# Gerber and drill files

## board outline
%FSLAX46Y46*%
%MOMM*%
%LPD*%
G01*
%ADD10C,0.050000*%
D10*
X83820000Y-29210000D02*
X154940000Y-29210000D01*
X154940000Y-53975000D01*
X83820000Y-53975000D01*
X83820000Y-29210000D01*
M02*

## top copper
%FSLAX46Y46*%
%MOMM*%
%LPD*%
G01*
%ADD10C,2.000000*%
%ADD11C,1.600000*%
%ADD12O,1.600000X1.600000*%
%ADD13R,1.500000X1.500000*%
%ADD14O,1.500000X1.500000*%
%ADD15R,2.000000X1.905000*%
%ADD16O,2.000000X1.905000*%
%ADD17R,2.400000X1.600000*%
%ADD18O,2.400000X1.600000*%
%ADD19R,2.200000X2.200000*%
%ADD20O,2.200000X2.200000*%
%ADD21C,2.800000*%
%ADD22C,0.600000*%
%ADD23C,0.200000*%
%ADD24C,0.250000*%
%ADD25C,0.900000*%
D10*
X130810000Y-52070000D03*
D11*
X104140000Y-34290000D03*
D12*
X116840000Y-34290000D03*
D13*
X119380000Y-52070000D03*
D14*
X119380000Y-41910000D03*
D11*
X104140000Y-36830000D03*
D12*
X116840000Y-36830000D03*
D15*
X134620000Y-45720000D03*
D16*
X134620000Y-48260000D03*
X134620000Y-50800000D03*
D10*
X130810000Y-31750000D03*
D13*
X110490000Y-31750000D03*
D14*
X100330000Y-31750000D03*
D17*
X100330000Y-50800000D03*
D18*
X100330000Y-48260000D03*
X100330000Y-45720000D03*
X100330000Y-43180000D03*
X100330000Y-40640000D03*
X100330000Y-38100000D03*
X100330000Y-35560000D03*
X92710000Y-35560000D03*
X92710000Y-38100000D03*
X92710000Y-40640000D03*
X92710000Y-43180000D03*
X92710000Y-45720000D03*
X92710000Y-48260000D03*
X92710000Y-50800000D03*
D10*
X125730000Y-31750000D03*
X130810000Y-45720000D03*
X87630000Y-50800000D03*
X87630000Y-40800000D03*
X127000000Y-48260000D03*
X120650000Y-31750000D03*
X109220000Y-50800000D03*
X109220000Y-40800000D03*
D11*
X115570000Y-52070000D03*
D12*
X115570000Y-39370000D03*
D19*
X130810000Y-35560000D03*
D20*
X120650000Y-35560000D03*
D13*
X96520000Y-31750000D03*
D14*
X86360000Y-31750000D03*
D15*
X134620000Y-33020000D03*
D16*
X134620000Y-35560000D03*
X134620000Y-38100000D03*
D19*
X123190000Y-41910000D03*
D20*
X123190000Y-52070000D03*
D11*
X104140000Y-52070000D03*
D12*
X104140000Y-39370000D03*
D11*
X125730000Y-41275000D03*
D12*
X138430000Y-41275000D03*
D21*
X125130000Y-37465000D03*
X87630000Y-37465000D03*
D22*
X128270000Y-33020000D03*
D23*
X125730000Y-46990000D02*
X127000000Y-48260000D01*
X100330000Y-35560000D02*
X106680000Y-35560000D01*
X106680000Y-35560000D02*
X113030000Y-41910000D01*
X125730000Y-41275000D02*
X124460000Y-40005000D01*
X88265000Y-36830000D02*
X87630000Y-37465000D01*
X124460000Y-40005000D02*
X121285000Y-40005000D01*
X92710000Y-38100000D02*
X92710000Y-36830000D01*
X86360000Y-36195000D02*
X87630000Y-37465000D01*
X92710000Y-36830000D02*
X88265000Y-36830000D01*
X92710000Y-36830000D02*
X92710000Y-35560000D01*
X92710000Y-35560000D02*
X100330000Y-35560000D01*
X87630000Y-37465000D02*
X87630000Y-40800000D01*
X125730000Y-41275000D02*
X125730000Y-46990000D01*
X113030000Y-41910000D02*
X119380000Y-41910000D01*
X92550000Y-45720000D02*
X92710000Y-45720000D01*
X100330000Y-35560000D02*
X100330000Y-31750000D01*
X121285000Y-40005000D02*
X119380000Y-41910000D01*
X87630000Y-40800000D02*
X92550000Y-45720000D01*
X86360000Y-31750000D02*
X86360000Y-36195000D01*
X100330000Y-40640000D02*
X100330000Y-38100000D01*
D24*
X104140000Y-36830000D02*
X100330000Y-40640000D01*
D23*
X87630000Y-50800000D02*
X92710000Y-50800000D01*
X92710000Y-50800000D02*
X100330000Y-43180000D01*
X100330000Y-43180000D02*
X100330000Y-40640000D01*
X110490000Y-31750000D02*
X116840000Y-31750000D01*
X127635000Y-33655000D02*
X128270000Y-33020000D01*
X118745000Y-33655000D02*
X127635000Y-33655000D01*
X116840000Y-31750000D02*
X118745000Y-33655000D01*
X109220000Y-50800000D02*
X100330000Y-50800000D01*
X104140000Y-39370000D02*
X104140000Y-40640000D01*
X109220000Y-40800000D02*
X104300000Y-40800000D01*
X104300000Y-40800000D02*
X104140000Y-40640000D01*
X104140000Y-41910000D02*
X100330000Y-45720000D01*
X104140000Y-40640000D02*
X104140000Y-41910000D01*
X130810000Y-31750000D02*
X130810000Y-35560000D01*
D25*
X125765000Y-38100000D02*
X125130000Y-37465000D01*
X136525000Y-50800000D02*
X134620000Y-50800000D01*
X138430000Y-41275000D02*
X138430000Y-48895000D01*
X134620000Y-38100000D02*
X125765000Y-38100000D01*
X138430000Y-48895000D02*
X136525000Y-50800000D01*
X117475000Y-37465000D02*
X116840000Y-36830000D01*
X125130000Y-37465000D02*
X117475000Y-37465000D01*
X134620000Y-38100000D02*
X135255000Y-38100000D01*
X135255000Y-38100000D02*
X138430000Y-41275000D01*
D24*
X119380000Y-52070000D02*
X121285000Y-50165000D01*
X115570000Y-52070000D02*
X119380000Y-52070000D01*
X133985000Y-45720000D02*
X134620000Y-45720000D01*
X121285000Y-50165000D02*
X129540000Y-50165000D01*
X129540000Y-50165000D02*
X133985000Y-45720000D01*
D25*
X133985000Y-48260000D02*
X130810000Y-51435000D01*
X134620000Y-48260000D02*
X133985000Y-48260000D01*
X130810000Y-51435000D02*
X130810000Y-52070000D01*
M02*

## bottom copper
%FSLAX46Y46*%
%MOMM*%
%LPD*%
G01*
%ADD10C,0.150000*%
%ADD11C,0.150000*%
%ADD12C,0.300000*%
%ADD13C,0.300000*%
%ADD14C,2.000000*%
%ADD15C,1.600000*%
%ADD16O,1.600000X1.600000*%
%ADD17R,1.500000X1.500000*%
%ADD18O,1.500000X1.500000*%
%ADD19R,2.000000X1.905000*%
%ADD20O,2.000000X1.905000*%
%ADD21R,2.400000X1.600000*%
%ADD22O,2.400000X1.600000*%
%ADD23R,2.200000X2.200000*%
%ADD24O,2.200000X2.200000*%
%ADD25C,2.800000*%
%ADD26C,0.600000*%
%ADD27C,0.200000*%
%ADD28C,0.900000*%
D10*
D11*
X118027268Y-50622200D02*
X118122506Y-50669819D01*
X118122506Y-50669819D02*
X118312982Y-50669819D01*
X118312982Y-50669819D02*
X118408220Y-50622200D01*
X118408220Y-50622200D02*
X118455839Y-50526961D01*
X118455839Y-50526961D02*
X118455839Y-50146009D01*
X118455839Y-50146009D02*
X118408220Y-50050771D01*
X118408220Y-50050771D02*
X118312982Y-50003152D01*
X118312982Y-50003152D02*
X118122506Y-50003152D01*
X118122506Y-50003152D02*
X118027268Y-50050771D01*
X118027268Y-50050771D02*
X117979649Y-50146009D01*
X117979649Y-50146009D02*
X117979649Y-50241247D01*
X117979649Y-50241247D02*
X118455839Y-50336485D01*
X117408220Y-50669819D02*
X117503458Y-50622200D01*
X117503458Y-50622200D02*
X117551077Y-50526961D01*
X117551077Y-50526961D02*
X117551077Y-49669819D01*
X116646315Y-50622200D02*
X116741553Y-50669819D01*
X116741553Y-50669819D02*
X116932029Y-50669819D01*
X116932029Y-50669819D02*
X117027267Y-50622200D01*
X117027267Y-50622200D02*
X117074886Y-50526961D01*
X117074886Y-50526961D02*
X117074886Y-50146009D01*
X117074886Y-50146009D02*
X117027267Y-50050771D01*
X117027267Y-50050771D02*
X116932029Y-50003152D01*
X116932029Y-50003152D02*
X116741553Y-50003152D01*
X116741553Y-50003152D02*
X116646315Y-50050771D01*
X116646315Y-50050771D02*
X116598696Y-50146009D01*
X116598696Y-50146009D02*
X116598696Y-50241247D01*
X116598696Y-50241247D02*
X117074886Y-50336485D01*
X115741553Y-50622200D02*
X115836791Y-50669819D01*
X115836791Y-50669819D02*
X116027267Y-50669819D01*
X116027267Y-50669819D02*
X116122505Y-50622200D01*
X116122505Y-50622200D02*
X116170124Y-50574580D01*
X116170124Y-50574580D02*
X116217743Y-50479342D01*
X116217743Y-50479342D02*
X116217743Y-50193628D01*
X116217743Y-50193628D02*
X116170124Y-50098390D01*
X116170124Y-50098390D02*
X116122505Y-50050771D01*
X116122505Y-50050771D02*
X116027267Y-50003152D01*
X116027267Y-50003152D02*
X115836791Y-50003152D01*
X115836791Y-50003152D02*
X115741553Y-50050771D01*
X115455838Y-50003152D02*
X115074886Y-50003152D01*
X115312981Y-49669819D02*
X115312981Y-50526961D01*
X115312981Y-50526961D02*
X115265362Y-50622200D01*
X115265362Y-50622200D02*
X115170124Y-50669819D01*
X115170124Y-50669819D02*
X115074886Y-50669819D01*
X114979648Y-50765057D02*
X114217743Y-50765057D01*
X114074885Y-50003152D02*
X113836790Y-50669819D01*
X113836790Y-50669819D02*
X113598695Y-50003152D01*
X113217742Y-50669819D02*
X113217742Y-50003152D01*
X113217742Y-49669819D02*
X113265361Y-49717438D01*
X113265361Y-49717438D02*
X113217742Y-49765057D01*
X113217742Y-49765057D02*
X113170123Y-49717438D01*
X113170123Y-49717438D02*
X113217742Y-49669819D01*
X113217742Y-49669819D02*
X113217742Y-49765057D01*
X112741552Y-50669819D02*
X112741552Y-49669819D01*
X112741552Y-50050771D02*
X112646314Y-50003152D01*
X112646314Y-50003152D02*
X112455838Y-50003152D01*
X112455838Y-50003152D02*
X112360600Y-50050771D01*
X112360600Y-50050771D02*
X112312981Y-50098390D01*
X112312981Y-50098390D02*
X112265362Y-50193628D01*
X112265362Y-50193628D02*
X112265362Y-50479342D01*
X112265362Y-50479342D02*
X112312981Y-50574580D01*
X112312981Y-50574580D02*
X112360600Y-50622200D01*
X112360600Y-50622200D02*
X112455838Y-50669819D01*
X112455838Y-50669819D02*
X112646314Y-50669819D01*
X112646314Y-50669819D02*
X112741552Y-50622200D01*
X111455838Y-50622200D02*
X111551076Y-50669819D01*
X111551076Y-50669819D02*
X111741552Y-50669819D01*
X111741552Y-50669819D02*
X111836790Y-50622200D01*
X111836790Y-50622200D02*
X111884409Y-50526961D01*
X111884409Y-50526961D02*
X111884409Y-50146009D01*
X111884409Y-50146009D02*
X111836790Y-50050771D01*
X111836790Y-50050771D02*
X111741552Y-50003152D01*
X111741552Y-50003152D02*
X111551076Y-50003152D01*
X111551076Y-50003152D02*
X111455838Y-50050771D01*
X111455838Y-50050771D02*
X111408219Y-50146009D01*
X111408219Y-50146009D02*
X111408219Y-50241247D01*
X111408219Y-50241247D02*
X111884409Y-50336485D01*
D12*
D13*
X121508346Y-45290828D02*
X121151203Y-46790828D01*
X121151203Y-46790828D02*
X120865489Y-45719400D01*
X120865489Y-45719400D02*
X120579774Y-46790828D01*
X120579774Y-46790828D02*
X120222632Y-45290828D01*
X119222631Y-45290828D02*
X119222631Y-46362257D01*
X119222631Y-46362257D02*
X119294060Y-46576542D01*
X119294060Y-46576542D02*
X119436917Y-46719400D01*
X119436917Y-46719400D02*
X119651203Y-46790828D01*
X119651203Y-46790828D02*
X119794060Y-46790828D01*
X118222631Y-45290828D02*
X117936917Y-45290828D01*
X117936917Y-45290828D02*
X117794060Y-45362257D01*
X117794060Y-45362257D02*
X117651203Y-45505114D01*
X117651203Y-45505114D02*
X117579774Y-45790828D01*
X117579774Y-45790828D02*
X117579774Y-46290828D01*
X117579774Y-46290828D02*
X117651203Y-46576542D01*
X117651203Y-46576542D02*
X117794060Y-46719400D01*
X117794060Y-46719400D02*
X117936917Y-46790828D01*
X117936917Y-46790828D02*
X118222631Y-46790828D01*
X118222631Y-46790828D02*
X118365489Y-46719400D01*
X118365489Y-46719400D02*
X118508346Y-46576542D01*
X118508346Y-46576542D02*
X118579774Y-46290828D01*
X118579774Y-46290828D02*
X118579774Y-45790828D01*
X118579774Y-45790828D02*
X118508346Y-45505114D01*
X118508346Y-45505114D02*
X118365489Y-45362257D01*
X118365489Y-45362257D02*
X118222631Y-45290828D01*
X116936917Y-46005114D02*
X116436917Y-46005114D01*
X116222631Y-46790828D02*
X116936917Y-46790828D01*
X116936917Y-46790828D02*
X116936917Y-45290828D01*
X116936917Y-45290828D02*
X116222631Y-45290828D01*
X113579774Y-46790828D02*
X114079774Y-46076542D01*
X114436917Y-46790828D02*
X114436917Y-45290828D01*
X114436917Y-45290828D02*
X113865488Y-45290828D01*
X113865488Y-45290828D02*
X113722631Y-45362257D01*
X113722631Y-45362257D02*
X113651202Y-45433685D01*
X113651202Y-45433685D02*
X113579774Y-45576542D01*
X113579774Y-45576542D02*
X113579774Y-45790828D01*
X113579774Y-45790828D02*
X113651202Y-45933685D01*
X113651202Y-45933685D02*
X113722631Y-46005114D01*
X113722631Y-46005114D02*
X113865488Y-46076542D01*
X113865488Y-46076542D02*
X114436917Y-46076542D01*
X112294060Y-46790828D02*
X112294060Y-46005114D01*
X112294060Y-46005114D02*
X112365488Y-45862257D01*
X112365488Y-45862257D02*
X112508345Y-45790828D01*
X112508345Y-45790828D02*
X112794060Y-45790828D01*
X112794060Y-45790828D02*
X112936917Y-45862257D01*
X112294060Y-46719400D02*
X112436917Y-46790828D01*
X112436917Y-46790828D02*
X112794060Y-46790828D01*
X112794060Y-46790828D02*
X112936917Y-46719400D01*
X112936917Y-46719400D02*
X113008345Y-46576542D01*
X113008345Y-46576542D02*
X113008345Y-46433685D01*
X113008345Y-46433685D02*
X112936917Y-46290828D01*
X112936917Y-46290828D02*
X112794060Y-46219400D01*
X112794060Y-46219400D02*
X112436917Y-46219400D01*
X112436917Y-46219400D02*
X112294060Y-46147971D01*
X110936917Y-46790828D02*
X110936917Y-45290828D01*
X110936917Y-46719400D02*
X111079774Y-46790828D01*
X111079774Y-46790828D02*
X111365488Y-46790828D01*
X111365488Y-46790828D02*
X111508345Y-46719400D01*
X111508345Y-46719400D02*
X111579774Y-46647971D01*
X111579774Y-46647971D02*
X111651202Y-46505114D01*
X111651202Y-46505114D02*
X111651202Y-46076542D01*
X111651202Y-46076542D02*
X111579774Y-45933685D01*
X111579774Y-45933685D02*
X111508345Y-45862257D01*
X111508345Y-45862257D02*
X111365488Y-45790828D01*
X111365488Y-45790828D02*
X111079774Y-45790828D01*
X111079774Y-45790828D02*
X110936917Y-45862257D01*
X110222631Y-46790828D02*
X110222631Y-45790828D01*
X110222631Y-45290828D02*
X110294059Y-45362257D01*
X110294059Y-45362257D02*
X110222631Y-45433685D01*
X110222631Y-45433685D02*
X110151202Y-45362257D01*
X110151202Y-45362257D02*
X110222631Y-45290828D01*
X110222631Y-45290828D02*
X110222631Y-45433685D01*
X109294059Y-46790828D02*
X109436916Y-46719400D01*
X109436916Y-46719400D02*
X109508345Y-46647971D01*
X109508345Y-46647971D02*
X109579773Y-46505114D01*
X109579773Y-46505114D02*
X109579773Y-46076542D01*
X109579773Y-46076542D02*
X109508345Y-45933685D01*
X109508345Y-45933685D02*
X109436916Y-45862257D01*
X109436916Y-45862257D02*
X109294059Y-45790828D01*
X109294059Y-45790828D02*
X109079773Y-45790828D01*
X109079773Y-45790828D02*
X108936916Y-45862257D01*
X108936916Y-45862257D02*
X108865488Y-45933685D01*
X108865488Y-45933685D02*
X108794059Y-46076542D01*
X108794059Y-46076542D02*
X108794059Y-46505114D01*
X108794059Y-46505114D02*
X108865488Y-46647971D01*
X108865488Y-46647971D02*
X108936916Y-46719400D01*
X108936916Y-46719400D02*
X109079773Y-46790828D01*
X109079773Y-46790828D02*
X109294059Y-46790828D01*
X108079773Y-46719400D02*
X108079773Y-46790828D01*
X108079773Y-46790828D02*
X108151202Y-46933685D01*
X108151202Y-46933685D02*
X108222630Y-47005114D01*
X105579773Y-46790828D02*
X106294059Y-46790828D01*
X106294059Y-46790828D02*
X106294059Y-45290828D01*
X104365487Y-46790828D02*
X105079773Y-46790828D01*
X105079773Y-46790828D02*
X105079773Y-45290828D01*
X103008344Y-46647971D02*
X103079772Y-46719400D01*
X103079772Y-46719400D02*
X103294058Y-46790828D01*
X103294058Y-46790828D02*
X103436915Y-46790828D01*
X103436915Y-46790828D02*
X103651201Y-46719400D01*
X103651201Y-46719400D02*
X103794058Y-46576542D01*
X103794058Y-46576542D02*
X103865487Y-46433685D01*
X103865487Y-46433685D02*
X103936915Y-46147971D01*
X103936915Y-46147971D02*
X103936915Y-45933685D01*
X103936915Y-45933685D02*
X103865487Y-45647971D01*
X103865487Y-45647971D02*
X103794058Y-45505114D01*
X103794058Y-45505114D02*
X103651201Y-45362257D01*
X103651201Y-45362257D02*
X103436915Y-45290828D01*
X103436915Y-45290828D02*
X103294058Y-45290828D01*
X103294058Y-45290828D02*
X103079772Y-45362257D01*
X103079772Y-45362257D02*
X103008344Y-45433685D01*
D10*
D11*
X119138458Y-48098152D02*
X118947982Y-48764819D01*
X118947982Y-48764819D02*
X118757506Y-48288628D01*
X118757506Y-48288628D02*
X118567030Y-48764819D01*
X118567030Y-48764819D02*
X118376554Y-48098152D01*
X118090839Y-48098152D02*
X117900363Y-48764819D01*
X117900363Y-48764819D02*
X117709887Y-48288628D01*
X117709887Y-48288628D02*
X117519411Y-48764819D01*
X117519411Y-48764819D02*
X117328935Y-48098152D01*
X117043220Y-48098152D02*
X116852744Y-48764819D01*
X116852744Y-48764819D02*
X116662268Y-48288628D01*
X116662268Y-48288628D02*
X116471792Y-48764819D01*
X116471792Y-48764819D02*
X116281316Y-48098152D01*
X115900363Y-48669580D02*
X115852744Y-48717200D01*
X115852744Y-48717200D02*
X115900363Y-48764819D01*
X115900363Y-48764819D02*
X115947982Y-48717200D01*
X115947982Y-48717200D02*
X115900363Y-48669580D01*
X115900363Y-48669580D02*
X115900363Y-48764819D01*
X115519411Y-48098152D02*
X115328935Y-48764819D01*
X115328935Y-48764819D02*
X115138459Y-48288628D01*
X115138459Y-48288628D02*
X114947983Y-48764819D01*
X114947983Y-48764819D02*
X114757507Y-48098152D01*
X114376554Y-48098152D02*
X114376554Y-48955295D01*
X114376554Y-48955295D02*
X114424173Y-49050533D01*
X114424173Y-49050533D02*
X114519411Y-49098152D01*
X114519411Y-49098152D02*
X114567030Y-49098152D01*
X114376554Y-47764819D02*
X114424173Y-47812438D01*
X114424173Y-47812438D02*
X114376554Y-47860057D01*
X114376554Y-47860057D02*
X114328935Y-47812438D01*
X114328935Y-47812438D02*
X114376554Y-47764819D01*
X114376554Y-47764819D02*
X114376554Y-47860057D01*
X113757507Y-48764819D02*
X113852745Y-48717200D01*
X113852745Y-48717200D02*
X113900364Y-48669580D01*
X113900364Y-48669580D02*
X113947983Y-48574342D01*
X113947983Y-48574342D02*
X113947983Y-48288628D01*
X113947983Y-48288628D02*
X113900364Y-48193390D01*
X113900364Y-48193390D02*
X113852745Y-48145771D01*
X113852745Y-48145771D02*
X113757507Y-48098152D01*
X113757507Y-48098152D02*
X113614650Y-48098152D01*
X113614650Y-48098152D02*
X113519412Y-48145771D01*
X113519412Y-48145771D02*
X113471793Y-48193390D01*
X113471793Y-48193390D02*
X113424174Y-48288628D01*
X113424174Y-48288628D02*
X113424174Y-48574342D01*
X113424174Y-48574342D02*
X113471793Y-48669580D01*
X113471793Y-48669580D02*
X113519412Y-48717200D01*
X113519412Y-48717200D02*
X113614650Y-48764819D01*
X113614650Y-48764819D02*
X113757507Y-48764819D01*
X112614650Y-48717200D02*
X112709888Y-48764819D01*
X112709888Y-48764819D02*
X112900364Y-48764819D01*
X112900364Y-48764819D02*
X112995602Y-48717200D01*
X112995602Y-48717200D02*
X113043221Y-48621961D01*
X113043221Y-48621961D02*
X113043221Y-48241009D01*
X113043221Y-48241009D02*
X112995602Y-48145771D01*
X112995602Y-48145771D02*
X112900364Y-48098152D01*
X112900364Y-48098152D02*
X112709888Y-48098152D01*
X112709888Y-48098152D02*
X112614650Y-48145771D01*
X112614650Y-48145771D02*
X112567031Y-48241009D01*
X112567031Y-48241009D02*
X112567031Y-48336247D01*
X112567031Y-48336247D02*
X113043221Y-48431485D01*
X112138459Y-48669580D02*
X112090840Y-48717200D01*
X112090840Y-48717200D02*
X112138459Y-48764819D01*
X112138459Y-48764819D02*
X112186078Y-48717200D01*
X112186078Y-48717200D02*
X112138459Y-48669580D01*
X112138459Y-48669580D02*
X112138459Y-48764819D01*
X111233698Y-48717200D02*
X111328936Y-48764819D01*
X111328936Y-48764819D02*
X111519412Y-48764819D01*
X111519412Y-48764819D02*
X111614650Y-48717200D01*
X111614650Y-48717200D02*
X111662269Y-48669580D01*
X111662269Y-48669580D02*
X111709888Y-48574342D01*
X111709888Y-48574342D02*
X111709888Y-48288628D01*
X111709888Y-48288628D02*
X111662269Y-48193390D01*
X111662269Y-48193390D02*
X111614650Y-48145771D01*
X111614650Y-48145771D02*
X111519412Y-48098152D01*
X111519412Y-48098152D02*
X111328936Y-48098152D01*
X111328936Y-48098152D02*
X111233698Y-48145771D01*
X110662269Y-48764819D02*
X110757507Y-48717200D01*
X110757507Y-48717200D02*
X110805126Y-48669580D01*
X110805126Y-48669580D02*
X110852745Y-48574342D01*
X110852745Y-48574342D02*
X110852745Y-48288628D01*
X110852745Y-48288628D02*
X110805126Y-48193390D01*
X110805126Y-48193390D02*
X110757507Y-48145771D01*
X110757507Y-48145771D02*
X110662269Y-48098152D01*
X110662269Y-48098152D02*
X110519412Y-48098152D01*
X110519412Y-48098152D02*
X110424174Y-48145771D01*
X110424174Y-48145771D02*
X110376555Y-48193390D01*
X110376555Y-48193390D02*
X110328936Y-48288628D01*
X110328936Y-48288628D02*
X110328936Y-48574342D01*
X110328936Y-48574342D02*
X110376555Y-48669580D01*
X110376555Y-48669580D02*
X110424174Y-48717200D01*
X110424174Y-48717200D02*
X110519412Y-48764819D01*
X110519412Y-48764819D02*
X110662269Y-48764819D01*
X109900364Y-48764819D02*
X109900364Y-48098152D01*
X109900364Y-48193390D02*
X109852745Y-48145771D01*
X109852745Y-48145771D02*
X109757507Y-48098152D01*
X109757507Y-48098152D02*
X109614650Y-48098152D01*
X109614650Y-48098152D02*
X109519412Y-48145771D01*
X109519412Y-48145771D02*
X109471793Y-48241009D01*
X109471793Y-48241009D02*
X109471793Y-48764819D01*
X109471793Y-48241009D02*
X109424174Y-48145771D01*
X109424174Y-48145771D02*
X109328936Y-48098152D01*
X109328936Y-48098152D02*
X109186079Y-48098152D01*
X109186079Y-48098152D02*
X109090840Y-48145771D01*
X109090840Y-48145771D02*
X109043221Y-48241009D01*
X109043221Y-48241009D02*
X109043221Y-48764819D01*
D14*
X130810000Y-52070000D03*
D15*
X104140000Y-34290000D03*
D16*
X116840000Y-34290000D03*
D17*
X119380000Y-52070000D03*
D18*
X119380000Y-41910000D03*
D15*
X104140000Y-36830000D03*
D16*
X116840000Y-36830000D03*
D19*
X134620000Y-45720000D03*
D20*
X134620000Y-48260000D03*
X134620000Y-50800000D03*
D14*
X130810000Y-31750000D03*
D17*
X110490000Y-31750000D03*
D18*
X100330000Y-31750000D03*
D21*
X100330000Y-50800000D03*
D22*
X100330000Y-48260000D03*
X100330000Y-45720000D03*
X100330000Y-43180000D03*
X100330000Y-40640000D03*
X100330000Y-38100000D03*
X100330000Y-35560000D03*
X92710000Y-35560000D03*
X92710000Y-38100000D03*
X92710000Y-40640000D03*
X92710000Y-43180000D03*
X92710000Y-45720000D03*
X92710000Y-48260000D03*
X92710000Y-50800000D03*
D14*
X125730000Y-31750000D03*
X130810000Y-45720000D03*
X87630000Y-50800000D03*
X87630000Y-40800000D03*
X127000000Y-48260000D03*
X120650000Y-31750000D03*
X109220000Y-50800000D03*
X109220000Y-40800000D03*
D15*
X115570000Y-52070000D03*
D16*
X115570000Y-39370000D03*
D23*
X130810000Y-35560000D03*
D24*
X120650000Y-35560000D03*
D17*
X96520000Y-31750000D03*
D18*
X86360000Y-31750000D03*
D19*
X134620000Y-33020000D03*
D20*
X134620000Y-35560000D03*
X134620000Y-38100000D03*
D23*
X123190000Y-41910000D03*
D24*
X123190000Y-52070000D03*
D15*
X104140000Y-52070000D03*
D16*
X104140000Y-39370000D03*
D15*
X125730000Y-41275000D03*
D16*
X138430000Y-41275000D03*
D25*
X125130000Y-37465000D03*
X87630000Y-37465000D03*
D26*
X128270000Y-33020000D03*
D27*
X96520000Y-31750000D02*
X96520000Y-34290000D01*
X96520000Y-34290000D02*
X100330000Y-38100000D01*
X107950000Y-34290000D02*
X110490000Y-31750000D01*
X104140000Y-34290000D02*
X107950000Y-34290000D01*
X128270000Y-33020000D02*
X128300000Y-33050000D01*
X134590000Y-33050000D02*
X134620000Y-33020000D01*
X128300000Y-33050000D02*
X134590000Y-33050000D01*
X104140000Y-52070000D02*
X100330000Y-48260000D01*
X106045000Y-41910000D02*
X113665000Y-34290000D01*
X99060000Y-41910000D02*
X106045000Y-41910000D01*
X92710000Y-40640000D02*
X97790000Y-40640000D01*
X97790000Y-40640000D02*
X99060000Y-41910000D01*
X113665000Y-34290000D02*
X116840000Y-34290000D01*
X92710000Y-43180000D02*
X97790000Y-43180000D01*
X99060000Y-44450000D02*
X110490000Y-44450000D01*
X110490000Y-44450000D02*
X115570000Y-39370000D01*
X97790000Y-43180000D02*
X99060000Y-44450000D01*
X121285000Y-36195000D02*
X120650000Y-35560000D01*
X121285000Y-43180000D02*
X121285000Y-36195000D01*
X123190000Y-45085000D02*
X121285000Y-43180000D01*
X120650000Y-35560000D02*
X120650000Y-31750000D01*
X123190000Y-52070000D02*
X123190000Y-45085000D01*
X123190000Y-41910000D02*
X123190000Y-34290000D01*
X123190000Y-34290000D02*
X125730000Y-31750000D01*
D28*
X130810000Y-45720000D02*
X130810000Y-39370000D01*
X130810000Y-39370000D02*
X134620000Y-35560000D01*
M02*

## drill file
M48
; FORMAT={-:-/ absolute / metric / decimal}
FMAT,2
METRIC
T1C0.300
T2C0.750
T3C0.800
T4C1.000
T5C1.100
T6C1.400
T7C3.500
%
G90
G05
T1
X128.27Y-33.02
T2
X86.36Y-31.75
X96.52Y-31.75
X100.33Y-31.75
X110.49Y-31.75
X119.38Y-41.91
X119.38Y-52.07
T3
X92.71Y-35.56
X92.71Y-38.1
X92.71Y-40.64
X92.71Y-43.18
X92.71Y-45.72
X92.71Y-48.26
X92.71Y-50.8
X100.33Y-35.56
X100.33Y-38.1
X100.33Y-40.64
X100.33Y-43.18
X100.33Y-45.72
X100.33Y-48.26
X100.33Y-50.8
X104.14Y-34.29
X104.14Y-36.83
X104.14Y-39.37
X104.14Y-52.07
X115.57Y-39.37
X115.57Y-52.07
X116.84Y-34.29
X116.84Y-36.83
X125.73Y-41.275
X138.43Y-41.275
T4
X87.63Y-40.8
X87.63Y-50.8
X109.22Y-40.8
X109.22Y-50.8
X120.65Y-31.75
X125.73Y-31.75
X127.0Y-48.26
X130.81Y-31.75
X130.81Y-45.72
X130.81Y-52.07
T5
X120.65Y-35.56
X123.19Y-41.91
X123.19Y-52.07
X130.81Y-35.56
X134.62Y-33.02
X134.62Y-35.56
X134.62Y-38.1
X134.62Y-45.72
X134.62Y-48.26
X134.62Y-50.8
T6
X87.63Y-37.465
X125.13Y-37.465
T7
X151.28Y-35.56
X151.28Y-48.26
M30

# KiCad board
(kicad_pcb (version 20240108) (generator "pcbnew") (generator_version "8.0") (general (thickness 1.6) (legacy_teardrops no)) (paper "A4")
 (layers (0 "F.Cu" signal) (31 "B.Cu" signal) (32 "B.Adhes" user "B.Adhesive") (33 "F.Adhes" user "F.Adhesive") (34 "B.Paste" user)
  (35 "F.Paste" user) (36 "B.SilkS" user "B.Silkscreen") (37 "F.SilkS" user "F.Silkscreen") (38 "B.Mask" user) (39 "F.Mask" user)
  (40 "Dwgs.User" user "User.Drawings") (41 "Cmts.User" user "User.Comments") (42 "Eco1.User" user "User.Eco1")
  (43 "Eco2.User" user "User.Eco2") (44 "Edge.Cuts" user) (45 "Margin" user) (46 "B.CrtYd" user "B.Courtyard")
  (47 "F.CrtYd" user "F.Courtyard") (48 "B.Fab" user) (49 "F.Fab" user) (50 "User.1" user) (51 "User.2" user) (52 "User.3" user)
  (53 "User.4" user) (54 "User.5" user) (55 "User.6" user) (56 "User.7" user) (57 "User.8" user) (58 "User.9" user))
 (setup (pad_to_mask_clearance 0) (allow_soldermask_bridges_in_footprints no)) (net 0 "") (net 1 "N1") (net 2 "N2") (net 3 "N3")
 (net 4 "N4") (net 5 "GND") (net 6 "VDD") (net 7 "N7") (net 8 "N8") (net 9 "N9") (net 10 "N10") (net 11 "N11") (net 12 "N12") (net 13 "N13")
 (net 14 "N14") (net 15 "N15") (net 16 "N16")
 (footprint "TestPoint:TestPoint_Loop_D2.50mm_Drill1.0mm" (layer "F.Cu") (at 130.81 52.07)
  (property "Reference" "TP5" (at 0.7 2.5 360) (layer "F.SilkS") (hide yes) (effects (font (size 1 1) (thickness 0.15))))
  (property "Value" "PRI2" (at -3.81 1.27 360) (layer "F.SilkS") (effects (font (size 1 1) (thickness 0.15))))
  (pad "1" thru_hole circle (at 0 0) (size 2 2) (drill 1) (layers "*.Cu" "*.Mask") (remove_unused_layers no) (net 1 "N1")))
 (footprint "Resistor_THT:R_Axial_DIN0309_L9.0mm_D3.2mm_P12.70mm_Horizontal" (layer "F.Cu") (at 104.14 34.29)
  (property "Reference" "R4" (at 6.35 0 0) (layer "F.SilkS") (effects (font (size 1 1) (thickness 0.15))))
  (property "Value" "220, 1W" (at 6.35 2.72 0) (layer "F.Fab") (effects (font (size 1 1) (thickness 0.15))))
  (pad "1" thru_hole circle (at 0 0) (size 1.6 1.6) (drill 0.8) (layers "*.Cu" "*.Mask") (remove_unused_layers no) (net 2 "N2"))
  (pad "2" thru_hole oval (at 12.7 0) (size 1.6 1.6) (drill 0.8) (layers "*.Cu" "*.Mask") (remove_unused_layers no) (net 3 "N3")))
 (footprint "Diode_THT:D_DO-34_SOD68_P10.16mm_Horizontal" (layer "F.Cu") (at 119.38 52.07 90)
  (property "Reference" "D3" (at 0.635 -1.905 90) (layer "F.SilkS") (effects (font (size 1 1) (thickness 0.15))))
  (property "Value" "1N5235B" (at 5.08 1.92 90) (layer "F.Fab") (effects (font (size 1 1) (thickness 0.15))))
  (pad "1" thru_hole rect (at 0 0 90) (size 1.5 1.5) (drill 0.75) (layers "*.Cu" "*.Mask") (remove_unused_layers no) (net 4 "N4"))
  (pad "2" thru_hole oval (at 10.16 0 90) (size 1.5 1.5) (drill 0.75) (layers "*.Cu" "*.Mask") (remove_unused_layers no) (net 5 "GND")))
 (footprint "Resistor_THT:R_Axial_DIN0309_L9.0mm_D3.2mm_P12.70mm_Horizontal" (layer "F.Cu") (at 104.14 36.83)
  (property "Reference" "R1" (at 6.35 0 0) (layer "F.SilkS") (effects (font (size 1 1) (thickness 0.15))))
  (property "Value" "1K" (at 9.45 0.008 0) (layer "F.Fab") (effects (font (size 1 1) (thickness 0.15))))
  (pad "1" thru_hole circle (at 0 0) (size 1.6 1.6) (drill 0.8) (layers "*.Cu" "*.Mask") (remove_unused_layers no) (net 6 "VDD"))
  (pad "2" thru_hole oval (at 12.7 0) (size 1.6 1.6) (drill 0.8) (layers "*.Cu" "*.Mask") (remove_unused_layers no) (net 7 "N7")))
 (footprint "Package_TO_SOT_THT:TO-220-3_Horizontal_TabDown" (layer "F.Cu") (at 134.62 45.72 -90)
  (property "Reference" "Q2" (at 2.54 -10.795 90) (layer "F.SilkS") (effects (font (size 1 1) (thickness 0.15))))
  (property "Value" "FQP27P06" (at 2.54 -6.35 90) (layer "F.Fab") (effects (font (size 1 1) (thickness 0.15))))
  (pad "" np_thru_hole circle (at 2.54 -16.66 270) (size 3.5 3.5) (drill 3.5) (layers "*.Cu" "*.Mask"))
  (pad "1" thru_hole rect (at 0 0 270) (size 1.905 2) (drill 1.1) (layers "*.Cu" "*.Mask") (remove_unused_layers no) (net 4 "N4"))
  (pad "2" thru_hole oval (at 2.54 0 270) (size 1.905 2) (drill 1.1) (layers "*.Cu" "*.Mask") (remove_unused_layers no) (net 1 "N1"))
  (pad "3" thru_hole oval (at 5.08 0 270) (size 1.905 2) (drill 1.1) (layers "*.Cu" "*.Mask") (remove_unused_layers no) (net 7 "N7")))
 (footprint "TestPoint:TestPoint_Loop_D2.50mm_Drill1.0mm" (layer "F.Cu") (at 130.81 31.75)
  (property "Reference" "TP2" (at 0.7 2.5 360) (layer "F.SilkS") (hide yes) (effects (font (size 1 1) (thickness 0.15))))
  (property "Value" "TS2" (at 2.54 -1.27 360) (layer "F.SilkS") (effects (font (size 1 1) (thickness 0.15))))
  (pad "1" thru_hole circle (at 0 0) (size 2 2) (drill 1) (layers "*.Cu" "*.Mask") (remove_unused_layers no) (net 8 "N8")))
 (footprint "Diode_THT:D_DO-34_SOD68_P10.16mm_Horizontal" (layer "F.Cu") (at 110.49 31.75 180)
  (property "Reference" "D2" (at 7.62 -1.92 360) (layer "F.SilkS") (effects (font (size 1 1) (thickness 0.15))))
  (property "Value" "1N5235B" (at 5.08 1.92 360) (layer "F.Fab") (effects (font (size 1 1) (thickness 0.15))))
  (pad "1" thru_hole rect (at 0 0 180) (size 1.5 1.5) (drill 0.75) (layers "*.Cu" "*.Mask") (remove_unused_layers no) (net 2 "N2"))
  (pad "2" thru_hole oval (at 10.16 0 180) (size 1.5 1.5) (drill 0.75) (layers "*.Cu" "*.Mask") (remove_unused_layers no) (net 5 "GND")))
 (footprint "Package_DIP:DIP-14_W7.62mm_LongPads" (layer "F.Cu") (at 100.33 50.8 180)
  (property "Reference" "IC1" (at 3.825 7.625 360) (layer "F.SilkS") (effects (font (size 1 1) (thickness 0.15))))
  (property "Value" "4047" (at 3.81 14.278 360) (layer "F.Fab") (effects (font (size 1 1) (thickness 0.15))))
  (pad "1" thru_hole rect (at 0 0 180) (size 2.4 1.6) (drill 0.8) (layers "*.Cu" "*.Mask") (remove_unused_layers no) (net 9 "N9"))
  (pad "2" thru_hole oval (at 0 2.54 180) (size 2.4 1.6) (drill 0.8) (layers "*.Cu" "*.Mask") (remove_unused_layers no) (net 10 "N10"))
  (pad "3" thru_hole oval (at 0 5.08 180) (size 2.4 1.6) (drill 0.8) (layers "*.Cu" "*.Mask") (remove_unused_layers no) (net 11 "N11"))
  (pad "4" thru_hole oval (at 0 7.62 180) (size 2.4 1.6) (drill 0.8) (layers "*.Cu" "*.Mask") (remove_unused_layers no) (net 6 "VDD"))
  (pad "5" thru_hole oval (at 0 10.16 180) (size 2.4 1.6) (drill 0.8) (layers "*.Cu" "*.Mask") (remove_unused_layers no) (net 6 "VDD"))
  (pad "6" thru_hole oval (at 0 12.7 180) (size 2.4 1.6) (drill 0.8) (layers "*.Cu" "*.Mask") (remove_unused_layers no) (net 6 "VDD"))
  (pad "7" thru_hole oval (at 0 15.24 180) (size 2.4 1.6) (drill 0.8) (layers "*.Cu" "*.Mask") (remove_unused_layers no) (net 5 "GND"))
  (pad "8" thru_hole oval (at 7.62 15.24 180) (size 2.4 1.6) (drill 0.8) (layers "*.Cu" "*.Mask") (remove_unused_layers no) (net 5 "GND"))
  (pad "9" thru_hole oval (at 7.62 12.7 180) (size 2.4 1.6) (drill 0.8) (layers "*.Cu" "*.Mask") (remove_unused_layers no) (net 5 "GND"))
  (pad "10" thru_hole oval (at 7.62 10.16 180) (size 2.4 1.6) (drill 0.8) (layers "*.Cu" "*.Mask") (remove_unused_layers no) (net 3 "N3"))
  (pad "11" thru_hole oval (at 7.62 7.62 180) (size 2.4 1.6) (drill 0.8) (layers "*.Cu" "*.Mask") (remove_unused_layers no) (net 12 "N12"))
  (pad "12" thru_hole oval (at 7.62 5.08 180) (size 2.4 1.6) (drill 0.8) (layers "*.Cu" "*.Mask") (remove_unused_layers no) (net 5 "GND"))
  (pad "13" thru_hole oval (at 7.62 2.54 180) (size 2.4 1.6) (drill 0.8) (layers "*.Cu" "*.Mask") (remove_unused_layers no) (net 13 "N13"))
  (pad "14" thru_hole oval (at 7.62 0 180) (size 2.4 1.6) (drill 0.8) (layers "*.Cu" "*.Mask") (remove_unused_layers no) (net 6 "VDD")))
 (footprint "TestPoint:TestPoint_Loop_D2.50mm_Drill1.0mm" (layer "F.Cu") (at 125.73 31.75 90)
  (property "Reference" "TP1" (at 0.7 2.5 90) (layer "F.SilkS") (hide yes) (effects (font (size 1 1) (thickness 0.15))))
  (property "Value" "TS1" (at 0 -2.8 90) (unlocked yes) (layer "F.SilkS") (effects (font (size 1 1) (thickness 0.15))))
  (pad "1" thru_hole circle (at 0 0 90) (size 2 2) (drill 1) (layers "*.Cu" "*.Mask") (remove_unused_layers no) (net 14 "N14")))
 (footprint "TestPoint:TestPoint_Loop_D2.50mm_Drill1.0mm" (layer "F.Cu") (at 130.81 45.72)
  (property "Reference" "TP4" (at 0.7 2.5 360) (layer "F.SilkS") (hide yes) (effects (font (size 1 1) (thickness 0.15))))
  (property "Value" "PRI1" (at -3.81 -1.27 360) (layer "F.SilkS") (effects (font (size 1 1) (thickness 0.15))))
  (pad "1" thru_hole circle (at 0 0) (size 2 2) (drill 1) (layers "*.Cu" "*.Mask") (remove_unused_layers no) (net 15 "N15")))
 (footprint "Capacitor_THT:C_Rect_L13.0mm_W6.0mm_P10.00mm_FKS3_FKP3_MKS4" (layer "F.Cu") (at 87.63 50.8 90)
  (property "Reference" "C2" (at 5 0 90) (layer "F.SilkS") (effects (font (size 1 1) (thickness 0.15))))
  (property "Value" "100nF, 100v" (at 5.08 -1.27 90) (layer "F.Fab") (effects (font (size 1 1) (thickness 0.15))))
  (pad "1" thru_hole circle (at 0 0 90) (size 2 2) (drill 1) (layers "*.Cu" "*.Mask") (remove_unused_layers no) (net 6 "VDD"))
  (pad "2" thru_hole circle (at 10 0 90) (size 2 2) (drill 1) (layers "*.Cu" "*.Mask") (remove_unused_layers no) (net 5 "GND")))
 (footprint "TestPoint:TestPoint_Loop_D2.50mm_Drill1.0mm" (layer "F.Cu") (at 127 48.26)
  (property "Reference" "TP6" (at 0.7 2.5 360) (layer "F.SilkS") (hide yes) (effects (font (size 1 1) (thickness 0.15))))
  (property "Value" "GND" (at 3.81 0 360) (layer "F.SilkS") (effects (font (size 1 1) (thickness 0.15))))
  (pad "1" thru_hole circle (at 0 0) (size 2 2) (drill 1) (layers "*.Cu" "*.Mask") (remove_unused_layers no) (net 5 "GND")))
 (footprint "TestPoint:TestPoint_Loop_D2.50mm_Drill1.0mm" (layer "F.Cu") (at 120.65 31.75)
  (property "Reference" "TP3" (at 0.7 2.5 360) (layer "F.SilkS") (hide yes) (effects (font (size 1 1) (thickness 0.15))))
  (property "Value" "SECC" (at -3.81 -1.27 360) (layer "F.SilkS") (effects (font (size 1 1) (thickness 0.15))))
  (pad "1" thru_hole circle (at 0 0) (size 2 2) (drill 1) (layers "*.Cu" "*.Mask") (remove_unused_layers no) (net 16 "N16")))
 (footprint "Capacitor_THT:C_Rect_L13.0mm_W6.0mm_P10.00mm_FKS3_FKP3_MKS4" (layer "F.Cu") (at 109.22 50.8 90)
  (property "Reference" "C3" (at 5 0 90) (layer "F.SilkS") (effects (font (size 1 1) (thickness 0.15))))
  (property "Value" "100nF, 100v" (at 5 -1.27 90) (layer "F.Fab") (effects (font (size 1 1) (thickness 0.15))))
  (pad "1" thru_hole circle (at 0 0 90) (size 2 2) (drill 1) (layers "*.Cu" "*.Mask") (remove_unused_layers no) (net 9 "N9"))
  (pad "2" thru_hole circle (at 10 0 90) (size 2 2) (drill 1) (layers "*.Cu" "*.Mask") (remove_unused_layers no) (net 11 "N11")))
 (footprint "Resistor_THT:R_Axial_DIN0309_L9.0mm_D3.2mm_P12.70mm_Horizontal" (layer "F.Cu") (at 115.57 52.07 90)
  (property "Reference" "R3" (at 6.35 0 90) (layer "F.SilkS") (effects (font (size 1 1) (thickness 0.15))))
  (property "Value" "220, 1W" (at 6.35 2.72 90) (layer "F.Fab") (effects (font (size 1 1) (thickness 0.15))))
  (pad "1" thru_hole circle (at 0 0 90) (size 1.6 1.6) (drill 0.8) (layers "*.Cu" "*.Mask") (remove_unused_layers no) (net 4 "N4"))
  (pad "2" thru_hole oval (at 12.7 0 90) (size 1.6 1.6) (drill 0.8) (layers "*.Cu" "*.Mask") (remove_unused_layers no) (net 12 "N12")))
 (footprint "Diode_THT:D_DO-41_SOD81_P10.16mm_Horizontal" (layer "F.Cu") (at 130.81 35.56 180)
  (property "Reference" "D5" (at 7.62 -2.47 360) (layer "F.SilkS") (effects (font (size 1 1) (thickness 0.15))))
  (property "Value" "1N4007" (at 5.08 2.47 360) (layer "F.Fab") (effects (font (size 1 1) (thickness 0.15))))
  (pad "1" thru_hole rect (at 0 0 180) (size 2.2 2.2) (drill 1.1) (layers "*.Cu" "*.Mask") (remove_unused_layers no) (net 8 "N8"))
  (pad "2" thru_hole oval (at 10.16 0 180) (size 2.2 2.2) (drill 1.1) (layers "*.Cu" "*.Mask") (remove_unused_layers no) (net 16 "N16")))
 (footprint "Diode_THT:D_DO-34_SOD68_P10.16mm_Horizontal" (layer "F.Cu") (at 96.52 31.75 180)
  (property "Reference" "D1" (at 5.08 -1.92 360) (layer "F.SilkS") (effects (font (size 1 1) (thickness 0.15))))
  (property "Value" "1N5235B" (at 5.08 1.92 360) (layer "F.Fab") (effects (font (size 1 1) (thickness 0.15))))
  (pad "1" thru_hole rect (at 0 0 180) (size 1.5 1.5) (drill 0.75) (layers "*.Cu" "*.Mask") (remove_unused_layers no) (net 6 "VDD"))
  (pad "2" thru_hole oval (at 10.16 0 180) (size 1.5 1.5) (drill 0.75) (layers "*.Cu" "*.Mask") (remove_unused_layers no) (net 5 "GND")))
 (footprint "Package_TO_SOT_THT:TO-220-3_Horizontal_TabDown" (layer "F.Cu") (at 134.62 33.02 -90)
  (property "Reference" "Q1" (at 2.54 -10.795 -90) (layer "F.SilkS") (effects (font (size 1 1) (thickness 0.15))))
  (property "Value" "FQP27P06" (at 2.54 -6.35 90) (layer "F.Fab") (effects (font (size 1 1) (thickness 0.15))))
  (pad "" np_thru_hole circle (at 2.54 -16.66 270) (size 3.5 3.5) (drill 3.5) (layers "*.Cu" "*.Mask"))
  (pad "1" thru_hole rect (at 0 0 270) (size 1.905 2) (drill 1.1) (layers "*.Cu" "*.Mask") (remove_unused_layers no) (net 2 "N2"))
  (pad "2" thru_hole oval (at 2.54 0 270) (size 1.905 2) (drill 1.1) (layers "*.Cu" "*.Mask") (remove_unused_layers no) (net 15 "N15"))
  (pad "3" thru_hole oval (at 5.08 0 270) (size 1.905 2) (drill 1.1) (layers "*.Cu" "*.Mask") (remove_unused_layers no) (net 7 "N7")))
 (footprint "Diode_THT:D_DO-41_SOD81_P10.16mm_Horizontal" (layer "F.Cu") (at 123.19 41.91 -90)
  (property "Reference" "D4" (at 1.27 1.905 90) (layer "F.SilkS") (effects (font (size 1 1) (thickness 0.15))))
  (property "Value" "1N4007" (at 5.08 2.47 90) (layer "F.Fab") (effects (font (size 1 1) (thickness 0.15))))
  (pad "1" thru_hole rect (at 0 0 270) (size 2.2 2.2) (drill 1.1) (layers "*.Cu" "*.Mask") (remove_unused_layers no) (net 14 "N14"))
  (pad "2" thru_hole oval (at 10.16 0 270) (size 2.2 2.2) (drill 1.1) (layers "*.Cu" "*.Mask") (remove_unused_layers no) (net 16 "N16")))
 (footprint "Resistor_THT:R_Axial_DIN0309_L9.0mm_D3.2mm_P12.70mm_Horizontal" (layer "F.Cu") (at 104.14 52.07 90)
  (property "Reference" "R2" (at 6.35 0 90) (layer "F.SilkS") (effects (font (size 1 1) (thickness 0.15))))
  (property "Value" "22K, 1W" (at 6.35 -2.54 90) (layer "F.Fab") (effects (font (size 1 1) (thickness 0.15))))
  (pad "1" thru_hole circle (at 0 0 90) (size 1.6 1.6) (drill 0.8) (layers "*.Cu" "*.Mask") (remove_unused_layers no) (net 10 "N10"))
  (pad "2" thru_hole oval (at 12.7 0 90) (size 1.6 1.6) (drill 0.8) (layers "*.Cu" "*.Mask") (remove_unused_layers no) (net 11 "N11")))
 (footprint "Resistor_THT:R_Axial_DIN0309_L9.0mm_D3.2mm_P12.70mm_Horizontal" (layer "F.Cu") (at 125.73 41.275)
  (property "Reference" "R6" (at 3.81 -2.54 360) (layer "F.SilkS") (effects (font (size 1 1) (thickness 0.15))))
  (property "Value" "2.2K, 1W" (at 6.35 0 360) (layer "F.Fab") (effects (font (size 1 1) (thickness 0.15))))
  (pad "1" thru_hole circle (at 0 0) (size 1.6 1.6) (drill 0.8) (layers "*.Cu" "*.Mask") (remove_unused_layers no) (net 5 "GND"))
  (pad "2" thru_hole oval (at 12.7 0) (size 1.6 1.6) (drill 0.8) (layers "*.Cu" "*.Mask") (remove_unused_layers no) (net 7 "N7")))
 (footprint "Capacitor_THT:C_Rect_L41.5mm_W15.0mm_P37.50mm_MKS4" (layer "B.Cu") (at 125.13 37.465 180)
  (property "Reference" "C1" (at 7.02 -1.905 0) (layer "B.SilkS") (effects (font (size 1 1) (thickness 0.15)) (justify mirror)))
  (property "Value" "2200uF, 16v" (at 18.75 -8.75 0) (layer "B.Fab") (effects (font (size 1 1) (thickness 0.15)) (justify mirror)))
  (pad "1" thru_hole circle (at 0 0 180) (size 2.8 2.8) (drill 1.4) (layers "*.Cu" "*.Mask") (remove_unused_layers no) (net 7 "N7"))
  (pad "2" thru_hole circle (at 37.5 0 180) (size 2.8 2.8) (drill 1.4) (layers "*.Cu" "*.Mask") (remove_unused_layers no) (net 5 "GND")))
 (gr_rect (start 83.82 29.21) (end 154.94 53.975) (stroke (width 0.05) (type default)) (fill none) (layer "Edge.Cuts"))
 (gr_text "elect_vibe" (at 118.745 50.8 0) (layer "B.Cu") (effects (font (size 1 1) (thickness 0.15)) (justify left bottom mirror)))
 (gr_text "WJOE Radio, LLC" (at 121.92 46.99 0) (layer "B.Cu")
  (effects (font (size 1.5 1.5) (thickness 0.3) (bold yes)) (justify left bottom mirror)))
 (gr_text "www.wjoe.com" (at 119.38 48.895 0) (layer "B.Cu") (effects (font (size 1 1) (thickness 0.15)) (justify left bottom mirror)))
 (segment (start 125.73 46.99) (end 127 48.26) (width 0.2) (layer "F.Cu") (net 5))
 (segment (start 100.33 35.56) (end 106.68 35.56) (width 0.2) (layer "F.Cu") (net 5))
 (segment (start 106.68 35.56) (end 113.03 41.91) (width 0.2) (layer "F.Cu") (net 5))
 (segment (start 125.73 41.275) (end 124.46 40.005) (width 0.2) (layer "F.Cu") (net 5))
 (segment (start 88.265 36.83) (end 87.63 37.465) (width 0.2) (layer "F.Cu") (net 5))
 (segment (start 124.46 40.005) (end 121.285 40.005) (width 0.2) (layer "F.Cu") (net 5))
 (segment (start 92.71 38.1) (end 92.71 36.83) (width 0.2) (layer "F.Cu") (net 5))
 (segment (start 86.36 36.195) (end 87.63 37.465) (width 0.2) (layer "F.Cu") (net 5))
 (segment (start 92.71 36.83) (end 88.265 36.83) (width 0.2) (layer "F.Cu") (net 5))
 (segment (start 92.71 36.83) (end 92.71 35.56) (width 0.2) (layer "F.Cu") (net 5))
 (segment (start 92.71 35.56) (end 100.33 35.56) (width 0.2) (layer "F.Cu") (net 5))
 (segment (start 87.63 37.465) (end 87.63 40.8) (width 0.2) (layer "F.Cu") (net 5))
 (segment (start 125.73 41.275) (end 125.73 46.99) (width 0.2) (layer "F.Cu") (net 5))
 (segment (start 113.03 41.91) (end 119.38 41.91) (width 0.2) (layer "F.Cu") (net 5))
 (segment (start 92.55 45.72) (end 92.71 45.72) (width 0.2) (layer "F.Cu") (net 5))
 (segment (start 100.33 35.56) (end 100.33 31.75) (width 0.2) (layer "F.Cu") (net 5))
 (segment (start 121.285 40.005) (end 119.38 41.91) (width 0.2) (layer "F.Cu") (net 5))
 (segment (start 87.63 40.8) (end 92.55 45.72) (width 0.2) (layer "F.Cu") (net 5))
 (segment (start 86.36 31.75) (end 86.36 36.195) (width 0.2) (layer "F.Cu") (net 5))
 (segment (start 100.33 40.64) (end 100.33 38.1) (width 0.2) (layer "F.Cu") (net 6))
 (segment (start 104.14 36.83) (end 100.33 40.64) (width 0.25) (layer "F.Cu") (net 6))
 (segment (start 87.63 50.8) (end 92.71 50.8) (width 0.2) (layer "F.Cu") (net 6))
 (segment (start 92.71 50.8) (end 100.33 43.18) (width 0.2) (layer "F.Cu") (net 6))
 (segment (start 100.33 43.18) (end 100.33 40.64) (width 0.2) (layer "F.Cu") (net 6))
 (segment (start 96.52 31.75) (end 96.52 34.29) (width 0.2) (layer "B.Cu") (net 6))
 (segment (start 96.52 34.29) (end 100.33 38.1) (width 0.2) (layer "B.Cu") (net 6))
 (segment (start 110.49 31.75) (end 116.84 31.75) (width 0.2) (layer "F.Cu") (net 2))
 (segment (start 127.635 33.655) (end 128.27 33.02) (width 0.2) (layer "F.Cu") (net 2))
 (segment (start 118.745 33.655) (end 127.635 33.655) (width 0.2) (layer "F.Cu") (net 2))
 (segment (start 116.84 31.75) (end 118.745 33.655) (width 0.2) (layer "F.Cu") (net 2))
 (via (at 128.27 33.02) (size 0.6) (drill 0.3) (layers "F.Cu" "B.Cu") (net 2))
 (segment (start 107.95 34.29) (end 110.49 31.75) (width 0.2) (layer "B.Cu") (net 2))
 (segment (start 104.14 34.29) (end 107.95 34.29) (width 0.2) (layer "B.Cu") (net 2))
 (segment (start 128.27 33.02) (end 128.3 33.05) (width 0.2) (layer "B.Cu") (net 2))
 (segment (start 134.59 33.05) (end 134.62 33.02) (width 0.2) (layer "B.Cu") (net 2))
 (segment (start 128.3 33.05) (end 134.59 33.05) (width 0.2) (layer "B.Cu") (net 2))
 (segment (start 109.22 50.8) (end 100.33 50.8) (width 0.2) (layer "F.Cu") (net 9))
 (segment (start 104.14 39.37) (end 104.14 40.64) (width 0.2) (layer "F.Cu") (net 11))
 (segment (start 109.22 40.8) (end 104.3 40.8) (width 0.2) (layer "F.Cu") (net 11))
 (segment (start 104.3 40.8) (end 104.14 40.64) (width 0.2) (layer "F.Cu") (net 11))
 (segment (start 104.14 41.91) (end 100.33 45.72) (width 0.2) (layer "F.Cu") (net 11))
 (segment (start 104.14 40.64) (end 104.14 41.91) (width 0.2) (layer "F.Cu") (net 11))
 (segment (start 104.14 52.07) (end 100.33 48.26) (width 0.2) (layer "B.Cu") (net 10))
 (segment (start 106.045 41.91) (end 113.665 34.29) (width 0.2) (layer "B.Cu") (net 3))
 (segment (start 99.06 41.91) (end 106.045 41.91) (width 0.2) (layer "B.Cu") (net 3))
 (segment (start 92.71 40.64) (end 97.79 40.64) (width 0.2) (layer "B.Cu") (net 3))
 (segment (start 97.79 40.64) (end 99.06 41.91) (width 0.2) (layer "B.Cu") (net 3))
 (segment (start 113.665 34.29) (end 116.84 34.29) (width 0.2) (layer "B.Cu") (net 3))
 (segment (start 92.71 43.18) (end 97.79 43.18) (width 0.2) (layer "B.Cu") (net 12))
 (segment (start 99.06 44.45) (end 110.49 44.45) (width 0.2) (layer "B.Cu") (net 12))
 (segment (start 110.49 44.45) (end 115.57 39.37) (width 0.2) (layer "B.Cu") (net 12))
 (segment (start 97.79 43.18) (end 99.06 44.45) (width 0.2) (layer "B.Cu") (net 12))
 (segment (start 121.285 36.195) (end 120.65 35.56) (width 0.2) (layer "B.Cu") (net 16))
 (segment (start 121.285 43.18) (end 121.285 36.195) (width 0.2) (layer "B.Cu") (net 16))
 (segment (start 123.19 45.085) (end 121.285 43.18) (width 0.2) (layer "B.Cu") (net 16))
 (segment (start 120.65 35.56) (end 120.65 31.75) (width 0.2) (layer "B.Cu") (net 16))
 (segment (start 123.19 52.07) (end 123.19 45.085) (width 0.2) (layer "B.Cu") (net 16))
 (segment (start 123.19 41.91) (end 123.19 34.29) (width 0.2) (layer "B.Cu") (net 14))
 (segment (start 123.19 34.29) (end 125.73 31.75) (width 0.2) (layer "B.Cu") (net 14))
 (segment (start 130.81 31.75) (end 130.81 35.56) (width 0.2) (layer "F.Cu") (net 8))
 (segment (start 125.765 38.1) (end 125.13 37.465) (width 0.9) (layer "F.Cu") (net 7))
 (segment (start 136.525 50.8) (end 134.62 50.8) (width 0.9) (layer "F.Cu") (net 7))
 (segment (start 138.43 41.275) (end 138.43 48.895) (width 0.9) (layer "F.Cu") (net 7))
 (segment (start 134.62 38.1) (end 125.765 38.1) (width 0.9) (layer "F.Cu") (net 7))
 (segment (start 138.43 48.895) (end 136.525 50.8) (width 0.9) (layer "F.Cu") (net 7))
 (segment (start 117.475 37.465) (end 116.84 36.83) (width 0.9) (layer "F.Cu") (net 7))
 (segment (start 125.13 37.465) (end 117.475 37.465) (width 0.9) (layer "F.Cu") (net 7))
 (segment (start 134.62 38.1) (end 135.255 38.1) (width 0.9) (layer "F.Cu") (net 7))
 (segment (start 135.255 38.1) (end 138.43 41.275) (width 0.9) (layer "F.Cu") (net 7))
 (segment (start 119.38 52.07) (end 121.285 50.165) (width 0.25) (layer "F.Cu") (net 4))
 (segment (start 115.57 52.07) (end 119.38 52.07) (width 0.25) (layer "F.Cu") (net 4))
 (segment (start 133.985 45.72) (end 134.62 45.72) (width 0.25) (layer "F.Cu") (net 4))
 (segment (start 121.285 50.165) (end 129.54 50.165) (width 0.25) (layer "F.Cu") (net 4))
 (segment (start 129.54 50.165) (end 133.985 45.72) (width 0.25) (layer "F.Cu") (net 4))
 (segment (start 130.81 45.72) (end 130.81 39.37) (width 0.9) (layer "B.Cu") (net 15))
 (segment (start 130.81 39.37) (end 134.62 35.56) (width 0.9) (layer "B.Cu") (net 15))
 (segment (start 133.985 48.26) (end 130.81 51.435) (width 0.9) (layer "F.Cu") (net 1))
 (segment (start 134.62 48.26) (end 133.985 48.26) (width 0.9) (layer "F.Cu") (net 1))
 (segment (start 130.81 51.435) (end 130.81 52.07) (width 0.9) (layer "F.Cu") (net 1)))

